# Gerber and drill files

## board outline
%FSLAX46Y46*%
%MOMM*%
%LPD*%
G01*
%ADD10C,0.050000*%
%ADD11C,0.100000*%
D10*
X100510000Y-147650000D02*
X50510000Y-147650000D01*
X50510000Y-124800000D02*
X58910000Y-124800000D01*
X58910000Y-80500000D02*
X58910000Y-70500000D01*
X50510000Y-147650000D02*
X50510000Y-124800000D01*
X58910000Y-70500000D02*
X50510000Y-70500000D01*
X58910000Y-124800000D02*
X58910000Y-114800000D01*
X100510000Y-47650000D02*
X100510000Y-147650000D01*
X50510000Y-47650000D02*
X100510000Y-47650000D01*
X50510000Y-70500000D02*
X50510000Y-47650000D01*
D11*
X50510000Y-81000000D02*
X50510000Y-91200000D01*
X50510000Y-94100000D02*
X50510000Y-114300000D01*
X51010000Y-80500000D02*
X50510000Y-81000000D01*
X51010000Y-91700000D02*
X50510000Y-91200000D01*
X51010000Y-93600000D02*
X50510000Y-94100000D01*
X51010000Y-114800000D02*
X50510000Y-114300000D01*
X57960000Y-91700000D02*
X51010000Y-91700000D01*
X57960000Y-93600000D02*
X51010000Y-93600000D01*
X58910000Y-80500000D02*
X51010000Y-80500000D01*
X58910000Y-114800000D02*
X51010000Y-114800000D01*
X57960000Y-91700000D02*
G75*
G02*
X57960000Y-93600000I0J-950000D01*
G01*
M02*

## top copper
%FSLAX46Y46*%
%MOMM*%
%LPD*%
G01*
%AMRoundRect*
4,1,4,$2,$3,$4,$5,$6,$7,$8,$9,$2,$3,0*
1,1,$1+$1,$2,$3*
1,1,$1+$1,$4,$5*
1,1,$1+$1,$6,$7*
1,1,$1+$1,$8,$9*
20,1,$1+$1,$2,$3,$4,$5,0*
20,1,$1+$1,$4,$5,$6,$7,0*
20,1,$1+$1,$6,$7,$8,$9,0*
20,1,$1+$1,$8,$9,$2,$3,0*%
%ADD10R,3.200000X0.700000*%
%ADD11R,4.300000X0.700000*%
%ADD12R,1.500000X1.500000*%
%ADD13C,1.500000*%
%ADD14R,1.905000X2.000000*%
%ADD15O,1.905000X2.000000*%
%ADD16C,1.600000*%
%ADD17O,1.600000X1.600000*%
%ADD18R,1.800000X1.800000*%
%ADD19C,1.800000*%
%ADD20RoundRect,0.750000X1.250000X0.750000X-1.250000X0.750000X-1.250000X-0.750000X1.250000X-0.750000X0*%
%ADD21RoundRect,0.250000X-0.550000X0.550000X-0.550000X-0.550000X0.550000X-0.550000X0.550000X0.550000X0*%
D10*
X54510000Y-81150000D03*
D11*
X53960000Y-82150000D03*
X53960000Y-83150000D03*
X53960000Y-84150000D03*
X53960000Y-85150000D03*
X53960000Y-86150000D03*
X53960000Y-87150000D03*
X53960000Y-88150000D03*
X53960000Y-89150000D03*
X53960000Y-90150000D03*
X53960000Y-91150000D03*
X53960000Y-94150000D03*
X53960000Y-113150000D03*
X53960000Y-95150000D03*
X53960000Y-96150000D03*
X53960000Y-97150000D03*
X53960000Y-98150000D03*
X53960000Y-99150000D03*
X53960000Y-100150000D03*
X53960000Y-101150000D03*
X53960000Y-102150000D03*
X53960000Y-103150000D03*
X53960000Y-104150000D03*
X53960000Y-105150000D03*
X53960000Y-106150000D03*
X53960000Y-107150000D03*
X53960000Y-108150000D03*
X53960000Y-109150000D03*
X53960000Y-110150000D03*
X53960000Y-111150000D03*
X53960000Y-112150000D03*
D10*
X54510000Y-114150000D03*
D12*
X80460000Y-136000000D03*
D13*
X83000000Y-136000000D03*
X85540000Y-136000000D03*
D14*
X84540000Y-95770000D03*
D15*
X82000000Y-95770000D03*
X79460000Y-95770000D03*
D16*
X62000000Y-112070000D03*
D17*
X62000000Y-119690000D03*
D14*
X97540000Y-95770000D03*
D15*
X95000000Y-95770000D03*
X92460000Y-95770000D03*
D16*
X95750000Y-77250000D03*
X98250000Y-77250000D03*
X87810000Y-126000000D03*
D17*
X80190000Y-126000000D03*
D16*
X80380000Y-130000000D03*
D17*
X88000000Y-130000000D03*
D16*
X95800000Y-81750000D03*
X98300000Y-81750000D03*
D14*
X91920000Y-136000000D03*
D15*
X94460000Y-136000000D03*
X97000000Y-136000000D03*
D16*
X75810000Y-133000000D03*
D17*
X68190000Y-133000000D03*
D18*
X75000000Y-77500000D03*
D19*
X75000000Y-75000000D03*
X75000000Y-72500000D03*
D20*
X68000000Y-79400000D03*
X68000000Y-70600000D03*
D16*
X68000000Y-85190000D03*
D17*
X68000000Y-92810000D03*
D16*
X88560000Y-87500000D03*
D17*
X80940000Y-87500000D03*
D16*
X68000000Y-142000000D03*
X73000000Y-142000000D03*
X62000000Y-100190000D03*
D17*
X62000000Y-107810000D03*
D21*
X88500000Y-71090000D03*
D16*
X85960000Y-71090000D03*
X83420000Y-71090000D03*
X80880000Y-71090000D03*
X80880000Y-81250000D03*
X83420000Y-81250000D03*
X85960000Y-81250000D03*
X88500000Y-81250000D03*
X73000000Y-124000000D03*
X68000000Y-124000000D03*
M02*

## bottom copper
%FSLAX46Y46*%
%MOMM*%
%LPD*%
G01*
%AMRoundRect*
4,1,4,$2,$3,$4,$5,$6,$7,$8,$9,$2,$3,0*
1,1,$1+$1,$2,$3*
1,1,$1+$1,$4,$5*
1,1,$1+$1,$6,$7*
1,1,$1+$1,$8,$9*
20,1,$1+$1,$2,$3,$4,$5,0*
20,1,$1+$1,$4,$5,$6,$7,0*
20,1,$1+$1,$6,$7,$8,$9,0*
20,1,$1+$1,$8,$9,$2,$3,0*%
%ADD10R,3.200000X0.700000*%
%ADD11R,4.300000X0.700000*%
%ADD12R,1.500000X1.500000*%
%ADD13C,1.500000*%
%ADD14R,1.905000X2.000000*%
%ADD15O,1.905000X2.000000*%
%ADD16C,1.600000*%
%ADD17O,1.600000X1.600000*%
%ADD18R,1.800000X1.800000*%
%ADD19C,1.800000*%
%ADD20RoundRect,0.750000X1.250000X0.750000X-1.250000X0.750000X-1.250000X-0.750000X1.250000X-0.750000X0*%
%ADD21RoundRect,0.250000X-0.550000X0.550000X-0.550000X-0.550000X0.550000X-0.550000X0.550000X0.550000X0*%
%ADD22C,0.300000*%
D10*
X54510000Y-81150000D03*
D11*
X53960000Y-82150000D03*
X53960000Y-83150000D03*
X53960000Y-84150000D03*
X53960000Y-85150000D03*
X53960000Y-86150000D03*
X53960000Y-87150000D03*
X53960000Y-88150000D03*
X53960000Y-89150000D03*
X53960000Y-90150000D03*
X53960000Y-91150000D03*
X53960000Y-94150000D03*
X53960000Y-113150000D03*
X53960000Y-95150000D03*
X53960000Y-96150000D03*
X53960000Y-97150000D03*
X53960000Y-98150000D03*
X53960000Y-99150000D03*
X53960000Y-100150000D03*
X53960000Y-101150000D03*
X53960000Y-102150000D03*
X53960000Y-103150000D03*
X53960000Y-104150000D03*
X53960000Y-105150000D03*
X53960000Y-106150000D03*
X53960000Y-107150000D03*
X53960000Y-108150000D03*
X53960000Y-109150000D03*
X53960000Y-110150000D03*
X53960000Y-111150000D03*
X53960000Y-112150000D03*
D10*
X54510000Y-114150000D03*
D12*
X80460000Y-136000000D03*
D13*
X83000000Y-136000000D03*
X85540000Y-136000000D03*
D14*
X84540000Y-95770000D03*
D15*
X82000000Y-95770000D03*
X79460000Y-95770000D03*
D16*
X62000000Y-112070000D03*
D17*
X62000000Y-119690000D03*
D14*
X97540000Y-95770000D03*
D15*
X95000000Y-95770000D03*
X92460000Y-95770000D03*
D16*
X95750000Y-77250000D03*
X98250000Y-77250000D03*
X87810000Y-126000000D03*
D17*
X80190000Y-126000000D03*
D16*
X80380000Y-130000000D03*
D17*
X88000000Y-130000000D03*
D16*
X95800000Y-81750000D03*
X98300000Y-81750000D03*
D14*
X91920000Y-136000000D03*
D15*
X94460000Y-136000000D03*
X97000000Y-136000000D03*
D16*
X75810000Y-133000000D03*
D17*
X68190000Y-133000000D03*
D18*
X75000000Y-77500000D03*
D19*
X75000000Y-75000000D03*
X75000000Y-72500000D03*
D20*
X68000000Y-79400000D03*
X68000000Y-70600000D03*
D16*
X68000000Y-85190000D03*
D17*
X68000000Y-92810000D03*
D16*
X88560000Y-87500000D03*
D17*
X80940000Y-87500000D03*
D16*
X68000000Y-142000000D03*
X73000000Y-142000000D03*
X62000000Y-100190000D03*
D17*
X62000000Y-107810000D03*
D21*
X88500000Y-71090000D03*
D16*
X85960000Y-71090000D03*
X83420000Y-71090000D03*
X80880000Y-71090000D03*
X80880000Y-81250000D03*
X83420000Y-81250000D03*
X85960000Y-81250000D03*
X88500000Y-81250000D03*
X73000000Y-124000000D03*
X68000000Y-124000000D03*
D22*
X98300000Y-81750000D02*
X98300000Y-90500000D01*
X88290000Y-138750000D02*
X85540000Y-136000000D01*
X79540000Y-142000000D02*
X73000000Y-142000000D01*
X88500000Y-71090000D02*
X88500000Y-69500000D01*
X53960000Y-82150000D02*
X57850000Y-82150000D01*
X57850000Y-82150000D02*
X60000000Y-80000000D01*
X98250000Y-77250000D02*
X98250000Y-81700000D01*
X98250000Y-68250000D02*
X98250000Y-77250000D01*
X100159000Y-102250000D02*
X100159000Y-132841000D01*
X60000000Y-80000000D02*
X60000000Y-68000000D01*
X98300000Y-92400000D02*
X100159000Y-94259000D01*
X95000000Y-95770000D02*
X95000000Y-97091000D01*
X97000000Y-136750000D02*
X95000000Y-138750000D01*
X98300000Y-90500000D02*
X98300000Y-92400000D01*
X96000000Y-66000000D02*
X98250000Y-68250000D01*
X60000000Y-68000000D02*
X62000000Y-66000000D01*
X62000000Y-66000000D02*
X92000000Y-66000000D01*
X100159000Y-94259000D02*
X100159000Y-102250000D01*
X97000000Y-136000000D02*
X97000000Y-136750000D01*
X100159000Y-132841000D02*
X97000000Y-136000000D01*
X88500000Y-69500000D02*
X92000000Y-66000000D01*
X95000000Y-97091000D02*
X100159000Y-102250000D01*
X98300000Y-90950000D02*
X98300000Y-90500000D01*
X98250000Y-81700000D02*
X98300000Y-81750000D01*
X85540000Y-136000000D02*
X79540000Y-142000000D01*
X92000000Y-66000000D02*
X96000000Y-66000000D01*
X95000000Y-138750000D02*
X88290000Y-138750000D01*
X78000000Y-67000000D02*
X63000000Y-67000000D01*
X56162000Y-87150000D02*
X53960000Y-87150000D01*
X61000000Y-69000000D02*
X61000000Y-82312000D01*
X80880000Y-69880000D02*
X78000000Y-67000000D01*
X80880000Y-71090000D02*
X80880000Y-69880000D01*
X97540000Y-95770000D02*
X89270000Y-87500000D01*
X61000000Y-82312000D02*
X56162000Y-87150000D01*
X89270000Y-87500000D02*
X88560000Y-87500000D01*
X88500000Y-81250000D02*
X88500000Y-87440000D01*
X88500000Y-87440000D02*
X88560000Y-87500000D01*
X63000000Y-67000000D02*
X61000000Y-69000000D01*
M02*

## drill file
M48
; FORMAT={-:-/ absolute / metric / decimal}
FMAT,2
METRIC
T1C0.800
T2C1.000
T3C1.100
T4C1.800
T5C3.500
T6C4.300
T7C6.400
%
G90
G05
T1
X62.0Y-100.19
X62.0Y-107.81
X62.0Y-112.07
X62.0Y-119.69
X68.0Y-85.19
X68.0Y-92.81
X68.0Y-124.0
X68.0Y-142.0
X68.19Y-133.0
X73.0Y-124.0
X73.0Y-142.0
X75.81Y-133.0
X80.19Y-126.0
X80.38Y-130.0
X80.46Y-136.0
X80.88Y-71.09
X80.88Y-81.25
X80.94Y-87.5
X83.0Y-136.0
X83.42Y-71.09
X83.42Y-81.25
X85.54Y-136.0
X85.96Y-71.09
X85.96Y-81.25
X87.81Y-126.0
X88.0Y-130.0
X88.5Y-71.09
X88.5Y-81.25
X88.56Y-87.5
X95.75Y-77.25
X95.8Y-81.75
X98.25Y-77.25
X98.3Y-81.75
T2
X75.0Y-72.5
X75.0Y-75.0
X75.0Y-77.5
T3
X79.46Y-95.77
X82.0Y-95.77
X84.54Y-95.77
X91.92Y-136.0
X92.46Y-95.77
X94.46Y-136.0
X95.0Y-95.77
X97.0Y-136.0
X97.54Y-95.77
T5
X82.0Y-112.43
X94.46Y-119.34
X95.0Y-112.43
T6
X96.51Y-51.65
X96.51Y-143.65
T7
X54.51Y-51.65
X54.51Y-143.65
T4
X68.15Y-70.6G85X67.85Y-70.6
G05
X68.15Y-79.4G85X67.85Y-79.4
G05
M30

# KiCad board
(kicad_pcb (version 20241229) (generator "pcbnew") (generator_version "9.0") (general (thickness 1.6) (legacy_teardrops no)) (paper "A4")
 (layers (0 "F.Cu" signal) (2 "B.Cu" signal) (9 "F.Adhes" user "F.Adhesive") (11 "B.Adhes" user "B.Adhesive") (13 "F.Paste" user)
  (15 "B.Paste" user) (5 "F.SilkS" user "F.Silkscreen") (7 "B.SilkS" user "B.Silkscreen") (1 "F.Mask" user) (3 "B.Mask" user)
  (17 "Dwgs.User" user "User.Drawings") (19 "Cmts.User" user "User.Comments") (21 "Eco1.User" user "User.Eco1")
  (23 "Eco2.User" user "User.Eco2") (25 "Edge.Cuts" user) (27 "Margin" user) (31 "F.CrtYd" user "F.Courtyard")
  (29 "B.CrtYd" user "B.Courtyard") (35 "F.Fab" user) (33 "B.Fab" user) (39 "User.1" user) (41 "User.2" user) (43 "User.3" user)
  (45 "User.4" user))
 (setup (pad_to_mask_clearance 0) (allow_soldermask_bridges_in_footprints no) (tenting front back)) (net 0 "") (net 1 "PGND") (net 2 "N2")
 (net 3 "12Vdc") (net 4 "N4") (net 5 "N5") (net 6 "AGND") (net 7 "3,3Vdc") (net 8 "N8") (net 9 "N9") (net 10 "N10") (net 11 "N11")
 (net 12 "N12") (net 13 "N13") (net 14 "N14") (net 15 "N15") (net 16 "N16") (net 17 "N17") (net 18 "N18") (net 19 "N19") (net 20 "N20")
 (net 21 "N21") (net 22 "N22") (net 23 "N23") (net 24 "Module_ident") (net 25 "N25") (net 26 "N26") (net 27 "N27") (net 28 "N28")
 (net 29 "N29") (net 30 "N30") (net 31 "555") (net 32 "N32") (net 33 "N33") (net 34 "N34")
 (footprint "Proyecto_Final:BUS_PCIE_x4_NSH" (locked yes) (layer "F.Cu") (at 53.96 81.15 -90)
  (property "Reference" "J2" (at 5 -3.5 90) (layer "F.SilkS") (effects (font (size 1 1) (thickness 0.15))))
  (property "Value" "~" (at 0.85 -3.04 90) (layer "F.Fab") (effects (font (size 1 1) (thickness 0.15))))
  (fp_line (start -0.15 3.45) (end 10.05 3.45) (stroke (width 0.1) (type solid)) (layer "Edge.Cuts"))
  (fp_line (start 12.95 3.45) (end 33.15 3.45) (stroke (width 0.1) (type solid)) (layer "Edge.Cuts"))
  (fp_line (start -0.65 2.95) (end -0.15 3.45) (stroke (width 0.1) (type solid)) (layer "Edge.Cuts"))
  (fp_line (start 10.55 2.95) (end 10.05 3.45) (stroke (width 0.1) (type solid)) (layer "Edge.Cuts"))
  (fp_line (start 12.45 2.95) (end 12.95 3.45) (stroke (width 0.1) (type solid)) (layer "Edge.Cuts"))
  (fp_line (start 33.65 2.95) (end 33.15 3.45) (stroke (width 0.1) (type solid)) (layer "Edge.Cuts"))
  (fp_line (start 10.55 -4) (end 10.55 2.95) (stroke (width 0.1) (type solid)) (layer "Edge.Cuts"))
  (fp_line (start 12.45 -4) (end 12.45 2.95) (stroke (width 0.1) (type solid)) (layer "Edge.Cuts"))
  (fp_line (start -0.65 -4.95) (end -0.65 2.95) (stroke (width 0.1) (type solid)) (layer "Edge.Cuts"))
  (fp_line (start 33.65 -4.95) (end 33.65 2.95) (stroke (width 0.1) (type solid)) (layer "Edge.Cuts"))
  (fp_arc (start 10.55 -4) (mid 11.5 -4.95) (end 12.45 -4) (stroke (width 0.1) (type solid)) (layer "Edge.Cuts"))
  (pad "1" connect rect (at 0 -0.55 270) (size 0.7 3.2) (layers "F.Cu" "F.Mask") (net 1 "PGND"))
  (pad "1" connect rect (at 0 -0.55 270) (size 0.7 3.2) (layers "B.Cu" "B.Mask") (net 1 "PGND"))
  (pad "2" connect rect (at 1 0 270) (size 0.7 4.3) (layers "F.Cu" "F.Mask") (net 1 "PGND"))
  (pad "2" connect rect (at 1 0 270) (size 0.7 4.3) (layers "B.Cu" "B.Mask") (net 1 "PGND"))
  (pad "2" connect rect (at 2 0 270) (size 0.7 4.3) (layers "F.Cu" "F.Mask") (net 1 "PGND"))
  (pad "2" connect rect (at 2 0 270) (size 0.7 4.3) (layers "B.Cu" "B.Mask") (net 1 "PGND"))
  (pad "2" connect rect (at 3 0 270) (size 0.7 4.3) (layers "F.Cu" "F.Mask") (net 1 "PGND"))
  (pad "2" connect rect (at 3 0 270) (size 0.7 4.3) (layers "B.Cu" "B.Mask") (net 1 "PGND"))
  (pad "2" connect rect (at 4 0 270) (size 0.7 4.3) (layers "F.Cu" "F.Mask") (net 1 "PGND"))
  (pad "2" connect rect (at 4 0 270) (size 0.7 4.3) (layers "B.Cu" "B.Mask") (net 1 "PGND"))
  (pad "3" connect rect (at 5 0 270) (size 0.7 4.3) (layers "F.Cu" "F.Mask") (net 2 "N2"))
  (pad "3" connect rect (at 5 0 270) (size 0.7 4.3) (layers "B.Cu" "B.Mask") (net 2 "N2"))
  (pad "4" connect rect (at 6 0 270) (size 0.7 4.3) (layers "F.Cu" "F.Mask") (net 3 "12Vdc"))
  (pad "4" connect rect (at 6 0 270) (size 0.7 4.3) (layers "B.Cu" "B.Mask") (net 3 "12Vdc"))
  (pad "4" connect rect (at 7 0 270) (size 0.7 4.3) (layers "F.Cu" "F.Mask") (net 3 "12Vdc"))
  (pad "4" connect rect (at 7 0 270) (size 0.7 4.3) (layers "B.Cu" "B.Mask") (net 3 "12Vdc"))
  (pad "4" connect rect (at 8 0 270) (size 0.7 4.3) (layers "F.Cu" "F.Mask") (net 3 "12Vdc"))
  (pad "4" connect rect (at 8 0 270) (size 0.7 4.3) (layers "B.Cu" "B.Mask") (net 3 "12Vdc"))
  (pad "5" connect rect (at 9 0 270) (size 0.7 4.3) (layers "F.Cu" "F.Mask") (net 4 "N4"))
  (pad "5" connect rect (at 9 0 270) (size 0.7 4.3) (layers "B.Cu" "B.Mask") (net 4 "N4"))
  (pad "6" connect rect (at 10 0 270) (size 0.7 4.3) (layers "F.Cu" "F.Mask") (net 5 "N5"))
  (pad "6" connect rect (at 10 0 270) (size 0.7 4.3) (layers "B.Cu" "B.Mask") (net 5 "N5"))
  (pad "7" connect rect (at 13 0 270) (size 0.7 4.3) (layers "F.Cu" "F.Mask") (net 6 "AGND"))
  (pad "7" connect rect (at 13 0 270) (size 0.7 4.3) (layers "B.Cu" "B.Mask") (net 6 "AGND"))
  (pad "7" connect rect (at 32 0 270) (size 0.7 4.3) (layers "F.Cu" "F.Mask") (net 6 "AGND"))
  (pad "7" connect rect (at 32 0 270) (size 0.7 4.3) (layers "B.Cu" "B.Mask") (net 6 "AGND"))
  (pad "8" connect rect (at 14 0 270) (size 0.7 4.3) (layers "F.Cu" "F.Mask") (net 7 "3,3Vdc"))
  (pad "8" connect rect (at 14 0 270) (size 0.7 4.3) (layers "B.Cu" "B.Mask") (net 7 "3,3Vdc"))
  (pad "9" connect rect (at 15 0 270) (size 0.7 4.3) (layers "F.Cu" "F.Mask") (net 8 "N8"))
  (pad "9" connect rect (at 15 0 270) (size 0.7 4.3) (layers "B.Cu" "B.Mask") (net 8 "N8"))
  (pad "10" connect rect (at 16 0 270) (size 0.7 4.3) (layers "F.Cu" "F.Mask") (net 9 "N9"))
  (pad "10" connect rect (at 16 0 270) (size 0.7 4.3) (layers "B.Cu" "B.Mask") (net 9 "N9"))
  (pad "11" connect rect (at 17 0 270) (size 0.7 4.3) (layers "F.Cu" "F.Mask") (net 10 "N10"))
  (pad "11" connect rect (at 17 0 270) (size 0.7 4.3) (layers "B.Cu" "B.Mask") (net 10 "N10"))
  (pad "12" connect rect (at 18 0 270) (size 0.7 4.3) (layers "F.Cu" "F.Mask") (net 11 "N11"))
  (pad "12" connect rect (at 18 0 270) (size 0.7 4.3) (layers "B.Cu" "B.Mask") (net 11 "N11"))
  (pad "13" connect rect (at 19 0 270) (size 0.7 4.3) (layers "F.Cu" "F.Mask") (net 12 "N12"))
  (pad "13" connect rect (at 19 0 270) (size 0.7 4.3) (layers "B.Cu" "B.Mask") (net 12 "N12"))
  (pad "14" connect rect (at 20 0 270) (size 0.7 4.3) (layers "F.Cu" "F.Mask") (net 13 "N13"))
  (pad "14" connect rect (at 20 0 270) (size 0.7 4.3) (layers "B.Cu" "B.Mask") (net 13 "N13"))
  (pad "15" connect rect (at 21 0 270) (size 0.7 4.3) (layers "F.Cu" "F.Mask") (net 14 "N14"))
  (pad "15" connect rect (at 21 0 270) (size 0.7 4.3) (layers "B.Cu" "B.Mask") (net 14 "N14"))
  (pad "16" connect rect (at 22 0 270) (size 0.7 4.3) (layers "F.Cu" "F.Mask") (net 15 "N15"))
  (pad "16" connect rect (at 22 0 270) (size 0.7 4.3) (layers "B.Cu" "B.Mask") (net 15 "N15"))
  (pad "17" connect rect (at 23 0 270) (size 0.7 4.3) (layers "F.Cu" "F.Mask") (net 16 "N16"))
  (pad "17" connect rect (at 23 0 270) (size 0.7 4.3) (layers "B.Cu" "B.Mask") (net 16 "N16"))
  (pad "18" connect rect (at 24 0 270) (size 0.7 4.3) (layers "F.Cu" "F.Mask") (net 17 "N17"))
  (pad "18" connect rect (at 24 0 270) (size 0.7 4.3) (layers "B.Cu" "B.Mask") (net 17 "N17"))
  (pad "19" connect rect (at 25 0 270) (size 0.7 4.3) (layers "F.Cu" "F.Mask") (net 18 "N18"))
  (pad "19" connect rect (at 25 0 270) (size 0.7 4.3) (layers "B.Cu" "B.Mask") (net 18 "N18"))
  (pad "20" connect rect (at 26 0 270) (size 0.7 4.3) (layers "F.Cu" "F.Mask") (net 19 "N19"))
  (pad "20" connect rect (at 26 0 270) (size 0.7 4.3) (layers "B.Cu" "B.Mask") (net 19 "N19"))
  (pad "21" connect rect (at 27 0 270) (size 0.7 4.3) (layers "F.Cu" "F.Mask") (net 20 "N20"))
  (pad "21" connect rect (at 27 0 270) (size 0.7 4.3) (layers "B.Cu" "B.Mask") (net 20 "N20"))
  (pad "22" connect rect (at 28 0 270) (size 0.7 4.3) (layers "F.Cu" "F.Mask") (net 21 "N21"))
  (pad "22" connect rect (at 28 0 270) (size 0.7 4.3) (layers "B.Cu" "B.Mask") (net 21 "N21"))
  (pad "23" connect rect (at 29 0 270) (size 0.7 4.3) (layers "F.Cu" "F.Mask") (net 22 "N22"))
  (pad "23" connect rect (at 29 0 270) (size 0.7 4.3) (layers "B.Cu" "B.Mask") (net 22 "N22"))
  (pad "24" connect rect (at 30 0 270) (size 0.7 4.3) (layers "F.Cu" "F.Mask") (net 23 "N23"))
  (pad "24" connect rect (at 30 0 270) (size 0.7 4.3) (layers "B.Cu" "B.Mask") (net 23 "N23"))
  (pad "25" connect rect (at 31 0 270) (size 0.7 4.3) (layers "F.Cu" "F.Mask") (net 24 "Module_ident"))
  (pad "25" connect rect (at 31 0 270) (size 0.7 4.3) (layers "B.Cu" "B.Mask") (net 24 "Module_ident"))
  (pad "26" connect rect (at 33 -0.55 270) (size 0.7 3.2) (layers "F.Cu" "F.Mask") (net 6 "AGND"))
  (pad "26" connect rect (at 33 -0.55 270) (size 0.7 3.2) (layers "B.Cu" "B.Mask") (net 6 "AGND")))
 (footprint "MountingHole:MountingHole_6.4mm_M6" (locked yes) (layer "F.Cu") (at 54.51 51.65)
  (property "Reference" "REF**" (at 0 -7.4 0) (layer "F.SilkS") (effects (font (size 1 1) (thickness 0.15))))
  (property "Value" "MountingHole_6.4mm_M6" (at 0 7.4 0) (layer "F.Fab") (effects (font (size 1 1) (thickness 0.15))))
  (pad "" np_thru_hole circle (at 0 0) (size 6.4 6.4) (drill 6.4) (layers "*.Cu" "*.Mask")))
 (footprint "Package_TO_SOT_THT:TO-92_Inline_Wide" (layer "F.Cu") (at 80.46 136)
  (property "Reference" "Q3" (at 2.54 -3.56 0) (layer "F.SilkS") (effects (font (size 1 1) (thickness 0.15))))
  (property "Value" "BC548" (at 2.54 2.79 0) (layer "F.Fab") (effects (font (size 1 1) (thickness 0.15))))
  (pad "1" thru_hole rect (at 0 0) (size 1.5 1.5) (drill 0.8) (layers "*.Cu" "*.Mask") (remove_unused_layers no) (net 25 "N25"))
  (pad "2" thru_hole circle (at 2.54 0) (size 1.5 1.5) (drill 0.8) (layers "*.Cu" "*.Mask") (remove_unused_layers no) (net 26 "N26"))
  (pad "3" thru_hole circle (at 5.08 0) (size 1.5 1.5) (drill 0.8) (layers "*.Cu" "*.Mask") (remove_unused_layers no) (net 1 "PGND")))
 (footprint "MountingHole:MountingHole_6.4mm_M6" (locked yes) (layer "F.Cu") (at 54.51 143.65)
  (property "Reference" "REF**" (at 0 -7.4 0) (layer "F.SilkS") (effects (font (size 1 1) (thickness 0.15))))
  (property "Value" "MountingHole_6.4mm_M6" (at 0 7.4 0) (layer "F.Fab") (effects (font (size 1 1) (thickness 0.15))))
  (pad "" np_thru_hole circle (at 0 0) (size 6.4 6.4) (drill 6.4) (layers "*.Cu" "*.Mask")))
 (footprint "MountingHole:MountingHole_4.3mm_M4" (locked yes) (layer "F.Cu") (at 96.51 143.65)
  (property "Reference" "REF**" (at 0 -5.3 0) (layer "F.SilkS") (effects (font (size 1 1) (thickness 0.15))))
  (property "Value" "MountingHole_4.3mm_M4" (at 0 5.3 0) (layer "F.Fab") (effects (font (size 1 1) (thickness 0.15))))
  (pad "" np_thru_hole circle (at 0 0) (size 4.3 4.3) (drill 4.3) (layers "*.Cu" "*.Mask")))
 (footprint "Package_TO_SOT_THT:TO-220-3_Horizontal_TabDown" (layer "F.Cu") (at 84.54 95.77 180)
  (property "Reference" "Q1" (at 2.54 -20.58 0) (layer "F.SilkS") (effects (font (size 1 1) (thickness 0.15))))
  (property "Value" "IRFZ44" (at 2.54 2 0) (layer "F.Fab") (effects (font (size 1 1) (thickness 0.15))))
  (pad "" np_thru_hole circle (at 2.54 -16.66 180) (size 3.5 3.5) (drill 3.5) (layers "*.Cu" "*.Mask"))
  (pad "1" thru_hole rect (at 0 0 180) (size 1.905 2) (drill 1.1) (layers "*.Cu" "*.Mask") (remove_unused_layers no) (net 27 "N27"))
  (pad "2" thru_hole oval (at 2.54 0 180) (size 1.905 2) (drill 1.1) (layers "*.Cu" "*.Mask") (remove_unused_layers no) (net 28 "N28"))
  (pad "3" thru_hole oval (at 5.08 0 180) (size 1.905 2) (drill 1.1) (layers "*.Cu" "*.Mask") (remove_unused_layers no) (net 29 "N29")))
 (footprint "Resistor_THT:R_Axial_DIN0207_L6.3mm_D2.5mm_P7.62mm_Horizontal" (layer "F.Cu") (at 62 112.07 -90)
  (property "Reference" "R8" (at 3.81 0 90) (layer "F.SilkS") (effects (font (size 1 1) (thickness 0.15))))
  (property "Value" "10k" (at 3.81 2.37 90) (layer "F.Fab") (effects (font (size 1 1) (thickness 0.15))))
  (pad "1" thru_hole circle (at 0 0 270) (size 1.6 1.6) (drill 0.8) (layers "*.Cu" "*.Mask") (remove_unused_layers no)
   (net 24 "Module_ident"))
  (pad "2" thru_hole oval (at 7.62 0 270) (size 1.6 1.6) (drill 0.8) (layers "*.Cu" "*.Mask") (remove_unused_layers no) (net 6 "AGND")))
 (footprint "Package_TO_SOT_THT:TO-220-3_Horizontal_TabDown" (layer "F.Cu") (at 97.54 95.77 180)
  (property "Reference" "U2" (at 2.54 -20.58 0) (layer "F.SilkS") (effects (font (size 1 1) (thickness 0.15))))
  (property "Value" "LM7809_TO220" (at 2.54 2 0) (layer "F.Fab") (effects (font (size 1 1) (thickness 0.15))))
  (pad "" np_thru_hole circle (at 2.54 -16.66 180) (size 3.5 3.5) (drill 3.5) (layers "*.Cu" "*.Mask"))
  (pad "1" thru_hole rect (at 0 0 180) (size 1.905 2) (drill 1.1) (layers "*.Cu" "*.Mask") (remove_unused_layers no) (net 3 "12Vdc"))
  (pad "2" thru_hole oval (at 2.54 0 180) (size 1.905 2) (drill 1.1) (layers "*.Cu" "*.Mask") (remove_unused_layers no) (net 1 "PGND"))
  (pad "3" thru_hole oval (at 5.08 0 180) (size 1.905 2) (drill 1.1) (layers "*.Cu" "*.Mask") (remove_unused_layers no) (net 27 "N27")))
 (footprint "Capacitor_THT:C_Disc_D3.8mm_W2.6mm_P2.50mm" (layer "F.Cu") (at 95.75 77.25)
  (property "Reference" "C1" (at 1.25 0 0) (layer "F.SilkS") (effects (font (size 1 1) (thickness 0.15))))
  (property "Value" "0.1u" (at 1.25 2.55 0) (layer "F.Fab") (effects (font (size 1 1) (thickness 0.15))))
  (pad "1" thru_hole circle (at 0 0) (size 1.6 1.6) (drill 0.8) (layers "*.Cu" "*.Mask") (remove_unused_layers no) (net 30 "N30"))
  (pad "2" thru_hole circle (at 2.5 0) (size 1.6 1.6) (drill 0.8) (layers "*.Cu" "*.Mask") (remove_unused_layers no) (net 1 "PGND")))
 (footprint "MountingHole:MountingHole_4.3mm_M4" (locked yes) (layer "F.Cu") (at 96.51 51.65)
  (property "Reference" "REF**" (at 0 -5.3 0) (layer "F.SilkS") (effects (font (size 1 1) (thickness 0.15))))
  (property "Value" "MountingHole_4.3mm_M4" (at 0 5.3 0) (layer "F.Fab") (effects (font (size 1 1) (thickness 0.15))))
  (pad "" np_thru_hole circle (at 0 0) (size 4.3 4.3) (drill 4.3) (layers "*.Cu" "*.Mask")))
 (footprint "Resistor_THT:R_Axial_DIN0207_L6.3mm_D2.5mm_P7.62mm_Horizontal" (layer "F.Cu") (at 87.81 126 180)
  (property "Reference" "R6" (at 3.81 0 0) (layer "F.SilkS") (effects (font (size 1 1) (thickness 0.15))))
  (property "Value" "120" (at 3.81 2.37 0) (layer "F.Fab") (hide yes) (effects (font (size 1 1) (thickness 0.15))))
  (pad "1" thru_hole circle (at 0 0 180) (size 1.6 1.6) (drill 0.8) (layers "*.Cu" "*.Mask") (remove_unused_layers no) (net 3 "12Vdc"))
  (pad "2" thru_hole oval (at 7.62 0 180) (size 1.6 1.6) (drill 0.8) (layers "*.Cu" "*.Mask") (remove_unused_layers no) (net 25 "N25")))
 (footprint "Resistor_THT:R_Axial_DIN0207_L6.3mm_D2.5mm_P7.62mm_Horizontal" (layer "F.Cu") (at 80.38 130)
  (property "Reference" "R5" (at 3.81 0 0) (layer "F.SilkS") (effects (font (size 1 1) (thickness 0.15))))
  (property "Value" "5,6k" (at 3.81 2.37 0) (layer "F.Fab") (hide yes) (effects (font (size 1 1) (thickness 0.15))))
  (pad "1" thru_hole circle (at 0 0) (size 1.6 1.6) (drill 0.8) (layers "*.Cu" "*.Mask") (remove_unused_layers no) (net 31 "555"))
  (pad "2" thru_hole oval (at 7.62 0) (size 1.6 1.6) (drill 0.8) (layers "*.Cu" "*.Mask") (remove_unused_layers no) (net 26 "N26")))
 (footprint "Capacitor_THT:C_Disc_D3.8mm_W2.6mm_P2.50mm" (layer "F.Cu") (at 95.8 81.75)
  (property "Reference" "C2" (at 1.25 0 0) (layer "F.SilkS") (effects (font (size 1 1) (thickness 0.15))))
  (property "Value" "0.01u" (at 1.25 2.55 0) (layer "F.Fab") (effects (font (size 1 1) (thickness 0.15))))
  (pad "1" thru_hole circle (at 0 0) (size 1.6 1.6) (drill 0.8) (layers "*.Cu" "*.Mask") (remove_unused_layers no) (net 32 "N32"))
  (pad "2" thru_hole circle (at 2.5 0) (size 1.6 1.6) (drill 0.8) (layers "*.Cu" "*.Mask") (remove_unused_layers no) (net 1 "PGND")))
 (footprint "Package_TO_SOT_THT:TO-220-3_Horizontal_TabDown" (layer "F.Cu") (at 91.92 136)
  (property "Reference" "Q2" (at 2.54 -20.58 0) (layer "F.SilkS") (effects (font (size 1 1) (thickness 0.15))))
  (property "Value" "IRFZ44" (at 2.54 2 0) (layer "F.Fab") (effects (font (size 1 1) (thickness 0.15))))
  (pad "" np_thru_hole circle (at 2.54 -16.66) (size 3.5 3.5) (drill 3.5) (layers "*.Cu" "*.Mask"))
  (pad "1" thru_hole rect (at 0 0) (size 1.905 2) (drill 1.1) (layers "*.Cu" "*.Mask") (remove_unused_layers no) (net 29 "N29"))
  (pad "2" thru_hole oval (at 2.54 0) (size 1.905 2) (drill 1.1) (layers "*.Cu" "*.Mask") (remove_unused_layers no) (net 25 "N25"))
  (pad "3" thru_hole oval (at 5.08 0) (size 1.905 2) (drill 1.1) (layers "*.Cu" "*.Mask") (remove_unused_layers no) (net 1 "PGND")))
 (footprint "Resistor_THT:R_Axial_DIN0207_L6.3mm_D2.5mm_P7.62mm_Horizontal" (layer "F.Cu") (at 75.81 133 180)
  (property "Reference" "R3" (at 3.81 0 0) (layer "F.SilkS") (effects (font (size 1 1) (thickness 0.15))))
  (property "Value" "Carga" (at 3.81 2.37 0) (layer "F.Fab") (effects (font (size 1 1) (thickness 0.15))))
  (pad "1" thru_hole circle (at 0 0 180) (size 1.6 1.6) (drill 0.8) (layers "*.Cu" "*.Mask") (remove_unused_layers no) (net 29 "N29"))
  (pad "2" thru_hole oval (at 7.62 0 180) (size 1.6 1.6) (drill 0.8) (layers "*.Cu" "*.Mask") (remove_unused_layers no) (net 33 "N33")))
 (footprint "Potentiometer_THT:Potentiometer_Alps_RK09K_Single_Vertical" (layer "F.Cu") (at 75 77.5 180)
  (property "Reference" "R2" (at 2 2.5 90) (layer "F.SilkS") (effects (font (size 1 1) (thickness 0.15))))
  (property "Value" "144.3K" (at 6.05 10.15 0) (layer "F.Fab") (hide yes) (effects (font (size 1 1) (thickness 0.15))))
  (pad "1" thru_hole rect (at 0 0 180) (size 1.8 1.8) (drill 1) (layers "*.Cu" "*.Mask") (remove_unused_layers no) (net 31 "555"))
  (pad "2" thru_hole circle (at 0 2.5 180) (size 1.8 1.8) (drill 1) (layers "*.Cu" "*.Mask") (remove_unused_layers no) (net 30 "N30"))
  (pad "3" thru_hole circle (at 0 5 180) (size 1.8 1.8) (drill 1) (layers "*.Cu" "*.Mask") (remove_unused_layers no))
  (pad "MP" thru_hole roundrect (at 7 -1.9 180) (size 4 3) (drill oval 2.1 1.8) (layers "*.Cu" "*.Mask") (remove_unused_layers no)
   (roundrect_rratio 0.25))
  (pad "MP" thru_hole roundrect (at 7 6.9 180) (size 4 3) (drill oval 2.1 1.8) (layers "*.Cu" "*.Mask") (remove_unused_layers no)
   (roundrect_rratio 0.25)))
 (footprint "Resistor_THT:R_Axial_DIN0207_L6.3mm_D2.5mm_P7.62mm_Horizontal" (layer "F.Cu") (at 68 85.19 -90)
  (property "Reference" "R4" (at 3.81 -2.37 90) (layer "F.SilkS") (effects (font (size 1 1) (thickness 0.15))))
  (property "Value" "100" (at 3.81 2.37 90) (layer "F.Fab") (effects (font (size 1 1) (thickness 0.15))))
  (pad "1" thru_hole circle (at 0 0 270) (size 1.6 1.6) (drill 0.8) (layers "*.Cu" "*.Mask") (remove_unused_layers no) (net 31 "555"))
  (pad "2" thru_hole oval (at 7.62 0 270) (size 1.6 1.6) (drill 0.8) (layers "*.Cu" "*.Mask") (remove_unused_layers no) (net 28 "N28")))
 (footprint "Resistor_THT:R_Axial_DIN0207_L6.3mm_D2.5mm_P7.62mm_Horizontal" (layer "F.Cu") (at 88.56 87.5 180)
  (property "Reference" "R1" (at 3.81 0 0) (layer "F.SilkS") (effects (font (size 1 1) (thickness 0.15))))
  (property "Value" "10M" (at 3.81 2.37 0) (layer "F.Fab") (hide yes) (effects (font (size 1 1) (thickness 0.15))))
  (pad "1" thru_hole circle (at 0 0 180) (size 1.6 1.6) (drill 0.8) (layers "*.Cu" "*.Mask") (remove_unused_layers no) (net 3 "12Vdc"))
  (pad "2" thru_hole oval (at 7.62 0 180) (size 1.6 1.6) (drill 0.8) (layers "*.Cu" "*.Mask") (remove_unused_layers no) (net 30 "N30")))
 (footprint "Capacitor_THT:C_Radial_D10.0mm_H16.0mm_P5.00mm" (layer "F.Cu") (at 68 142)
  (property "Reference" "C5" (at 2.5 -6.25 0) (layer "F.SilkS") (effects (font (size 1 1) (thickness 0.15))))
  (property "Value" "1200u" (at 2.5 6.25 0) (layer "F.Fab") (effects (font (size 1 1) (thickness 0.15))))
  (pad "1" thru_hole circle (at 0 0) (size 1.6 1.6) (drill 0.8) (layers "*.Cu" "*.Mask") (remove_unused_layers no) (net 33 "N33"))
  (pad "2" thru_hole circle (at 5 0) (size 1.6 1.6) (drill 0.8) (layers "*.Cu" "*.Mask") (remove_unused_layers no) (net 1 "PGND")))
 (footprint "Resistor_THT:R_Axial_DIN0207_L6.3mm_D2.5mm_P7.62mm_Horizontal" (layer "F.Cu") (at 62 100.19 -90)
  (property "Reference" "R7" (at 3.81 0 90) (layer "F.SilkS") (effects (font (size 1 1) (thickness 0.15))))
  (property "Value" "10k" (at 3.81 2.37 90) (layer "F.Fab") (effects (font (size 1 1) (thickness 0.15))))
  (pad "1" thru_hole circle (at 0 0 270) (size 1.6 1.6) (drill 0.8) (layers "*.Cu" "*.Mask") (remove_unused_layers no) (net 7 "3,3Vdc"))
  (pad "2" thru_hole oval (at 7.62 0 270) (size 1.6 1.6) (drill 0.8) (layers "*.Cu" "*.Mask") (remove_unused_layers no)
   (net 24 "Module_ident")))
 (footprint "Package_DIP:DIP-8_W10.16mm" (layer "F.Cu") (at 88.5 71.09 -90)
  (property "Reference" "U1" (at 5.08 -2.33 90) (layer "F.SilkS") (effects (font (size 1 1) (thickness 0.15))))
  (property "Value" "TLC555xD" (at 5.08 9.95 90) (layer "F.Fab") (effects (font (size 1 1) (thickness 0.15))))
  (pad "1" thru_hole roundrect (at 0 0 270) (size 1.6 1.6) (drill 0.8) (layers "*.Cu" "*.Mask") (remove_unused_layers no)
   (roundrect_rratio 0.15625) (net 1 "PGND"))
  (pad "2" thru_hole circle (at 0 2.54 270) (size 1.6 1.6) (drill 0.8) (layers "*.Cu" "*.Mask") (remove_unused_layers no) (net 30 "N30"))
  (pad "3" thru_hole circle (at 0 5.08 270) (size 1.6 1.6) (drill 0.8) (layers "*.Cu" "*.Mask") (remove_unused_layers no) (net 31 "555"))
  (pad "4" thru_hole circle (at 0 7.62 270) (size 1.6 1.6) (drill 0.8) (layers "*.Cu" "*.Mask") (remove_unused_layers no) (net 3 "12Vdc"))
  (pad "5" thru_hole circle (at 10.16 7.62 270) (size 1.6 1.6) (drill 0.8) (layers "*.Cu" "*.Mask") (remove_unused_layers no) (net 32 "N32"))
  (pad "6" thru_hole circle (at 10.16 5.08 270) (size 1.6 1.6) (drill 0.8) (layers "*.Cu" "*.Mask") (remove_unused_layers no) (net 30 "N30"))
  (pad "7" thru_hole circle (at 10.16 2.54 270) (size 1.6 1.6) (drill 0.8) (layers "*.Cu" "*.Mask") (remove_unused_layers no) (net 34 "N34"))
  (pad "8" thru_hole circle (at 10.16 0 270) (size 1.6 1.6) (drill 0.8) (layers "*.Cu" "*.Mask") (remove_unused_layers no) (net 3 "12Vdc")))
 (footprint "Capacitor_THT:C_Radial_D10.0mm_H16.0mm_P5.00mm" (layer "F.Cu") (at 73 124 180)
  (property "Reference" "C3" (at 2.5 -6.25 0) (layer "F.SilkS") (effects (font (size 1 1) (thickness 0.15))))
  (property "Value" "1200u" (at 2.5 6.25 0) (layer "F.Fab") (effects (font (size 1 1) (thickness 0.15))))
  (pad "1" thru_hole circle (at 0 0 180) (size 1.6 1.6) (drill 0.8) (layers "*.Cu" "*.Mask") (remove_unused_layers no) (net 27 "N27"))
  (pad "2" thru_hole circle (at 5 0 180) (size 1.6 1.6) (drill 0.8) (layers "*.Cu" "*.Mask") (remove_unused_layers no) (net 33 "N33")))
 (gr_line (start 100.51 147.65) (end 50.51 147.65) (stroke (width 0.05) (type solid)) (layer "Edge.Cuts"))
 (gr_line (start 50.51 124.8) (end 58.91 124.8) (stroke (width 0.05) (type solid)) (layer "Edge.Cuts"))
 (gr_line (start 58.91 80.5) (end 58.91 70.5) (stroke (width 0.05) (type solid)) (layer "Edge.Cuts"))
 (gr_line (start 50.51 147.65) (end 50.51 124.8) (stroke (width 0.05) (type solid)) (layer "Edge.Cuts"))
 (gr_line (start 58.91 70.5) (end 50.51 70.5) (stroke (width 0.05) (type solid)) (layer "Edge.Cuts"))
 (gr_line (start 58.91 124.8) (end 58.91 114.8) (stroke (width 0.05) (type solid)) (layer "Edge.Cuts"))
 (gr_line (start 100.51 47.65) (end 100.51 147.65) (stroke (width 0.05) (type solid)) (layer "Edge.Cuts"))
 (gr_line (start 50.51 47.65) (end 100.51 47.65) (stroke (width 0.05) (type solid)) (layer "Edge.Cuts"))
 (gr_line (start 50.51 70.5) (end 50.51 47.65) (stroke (width 0.05) (type solid)) (layer "Edge.Cuts"))
 (segment (start 98.3 81.75) (end 98.3 90.5) (width 0.3) (layer "B.Cu") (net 1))
 (segment (start 88.29 138.75) (end 85.54 136) (width 0.3) (layer "B.Cu") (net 1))
 (segment (start 79.54 142) (end 73 142) (width 0.3) (layer "B.Cu") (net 1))
 (segment (start 88.5 71.09) (end 88.5 69.5) (width 0.3) (layer "B.Cu") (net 1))
 (segment (start 53.96 82.15) (end 57.85 82.15) (width 0.3) (layer "B.Cu") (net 1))
 (segment (start 57.85 82.15) (end 60 80) (width 0.3) (layer "B.Cu") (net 1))
 (segment (start 98.25 77.25) (end 98.25 81.7) (width 0.3) (layer "B.Cu") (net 1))
 (segment (start 98.25 68.25) (end 98.25 77.25) (width 0.3) (layer "B.Cu") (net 1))
 (segment (start 100.159 102.25) (end 100.159 132.841) (width 0.3) (layer "B.Cu") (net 1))
 (segment (start 60 80) (end 60 68) (width 0.3) (layer "B.Cu") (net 1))
 (segment (start 98.3 92.4) (end 100.159 94.259) (width 0.3) (layer "B.Cu") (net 1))
 (segment (start 95 95.77) (end 95 97.091) (width 0.3) (layer "B.Cu") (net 1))
 (segment (start 97 136.75) (end 95 138.75) (width 0.3) (layer "B.Cu") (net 1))
 (segment (start 98.3 90.5) (end 98.3 92.4) (width 0.3) (layer "B.Cu") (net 1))
 (segment (start 96 66) (end 98.25 68.25) (width 0.3) (layer "B.Cu") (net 1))
 (segment (start 60 68) (end 62 66) (width 0.3) (layer "B.Cu") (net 1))
 (segment (start 62 66) (end 92 66) (width 0.3) (layer "B.Cu") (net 1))
 (segment (start 100.159 94.259) (end 100.159 102.25) (width 0.3) (layer "B.Cu") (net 1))
 (segment (start 97 136) (end 97 136.75) (width 0.3) (layer "B.Cu") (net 1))
 (segment (start 100.159 132.841) (end 97 136) (width 0.3) (layer "B.Cu") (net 1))
 (segment (start 88.5 69.5) (end 92 66) (width 0.3) (layer "B.Cu") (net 1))
 (segment (start 95 97.091) (end 100.159 102.25) (width 0.3) (layer "B.Cu") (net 1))
 (segment (start 98.3 90.95) (end 98.3 90.5) (width 0.3) (layer "B.Cu") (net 1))
 (segment (start 98.25 81.7) (end 98.3 81.75) (width 0.3) (layer "B.Cu") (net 1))
 (segment (start 85.54 136) (end 79.54 142) (width 0.3) (layer "B.Cu") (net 1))
 (segment (start 92 66) (end 96 66) (width 0.3) (layer "B.Cu") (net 1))
 (segment (start 95 138.75) (end 88.29 138.75) (width 0.3) (layer "B.Cu") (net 1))
 (segment (start 78 67) (end 63 67) (width 0.3) (layer "B.Cu") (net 3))
 (segment (start 56.162 87.15) (end 53.96 87.15) (width 0.3) (layer "B.Cu") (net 3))
 (segment (start 61 69) (end 61 82.312) (width 0.3) (layer "B.Cu") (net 3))
 (segment (start 80.88 69.88) (end 78 67) (width 0.3) (layer "B.Cu") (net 3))
 (segment (start 80.88 71.09) (end 80.88 69.88) (width 0.3) (layer "B.Cu") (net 3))
 (segment (start 97.54 95.77) (end 89.27 87.5) (width 0.3) (layer "B.Cu") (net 3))
 (segment (start 61 82.312) (end 56.162 87.15) (width 0.3) (layer "B.Cu") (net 3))
 (segment (start 89.27 87.5) (end 88.56 87.5) (width 0.3) (layer "B.Cu") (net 3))
 (segment (start 88.5 81.25) (end 88.5 87.44) (width 0.3) (layer "B.Cu") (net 3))
 (segment (start 88.5 87.44) (end 88.56 87.5) (width 0.3) (layer "B.Cu") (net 3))
 (segment (start 63 67) (end 61 69) (width 0.3) (layer "B.Cu") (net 3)))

